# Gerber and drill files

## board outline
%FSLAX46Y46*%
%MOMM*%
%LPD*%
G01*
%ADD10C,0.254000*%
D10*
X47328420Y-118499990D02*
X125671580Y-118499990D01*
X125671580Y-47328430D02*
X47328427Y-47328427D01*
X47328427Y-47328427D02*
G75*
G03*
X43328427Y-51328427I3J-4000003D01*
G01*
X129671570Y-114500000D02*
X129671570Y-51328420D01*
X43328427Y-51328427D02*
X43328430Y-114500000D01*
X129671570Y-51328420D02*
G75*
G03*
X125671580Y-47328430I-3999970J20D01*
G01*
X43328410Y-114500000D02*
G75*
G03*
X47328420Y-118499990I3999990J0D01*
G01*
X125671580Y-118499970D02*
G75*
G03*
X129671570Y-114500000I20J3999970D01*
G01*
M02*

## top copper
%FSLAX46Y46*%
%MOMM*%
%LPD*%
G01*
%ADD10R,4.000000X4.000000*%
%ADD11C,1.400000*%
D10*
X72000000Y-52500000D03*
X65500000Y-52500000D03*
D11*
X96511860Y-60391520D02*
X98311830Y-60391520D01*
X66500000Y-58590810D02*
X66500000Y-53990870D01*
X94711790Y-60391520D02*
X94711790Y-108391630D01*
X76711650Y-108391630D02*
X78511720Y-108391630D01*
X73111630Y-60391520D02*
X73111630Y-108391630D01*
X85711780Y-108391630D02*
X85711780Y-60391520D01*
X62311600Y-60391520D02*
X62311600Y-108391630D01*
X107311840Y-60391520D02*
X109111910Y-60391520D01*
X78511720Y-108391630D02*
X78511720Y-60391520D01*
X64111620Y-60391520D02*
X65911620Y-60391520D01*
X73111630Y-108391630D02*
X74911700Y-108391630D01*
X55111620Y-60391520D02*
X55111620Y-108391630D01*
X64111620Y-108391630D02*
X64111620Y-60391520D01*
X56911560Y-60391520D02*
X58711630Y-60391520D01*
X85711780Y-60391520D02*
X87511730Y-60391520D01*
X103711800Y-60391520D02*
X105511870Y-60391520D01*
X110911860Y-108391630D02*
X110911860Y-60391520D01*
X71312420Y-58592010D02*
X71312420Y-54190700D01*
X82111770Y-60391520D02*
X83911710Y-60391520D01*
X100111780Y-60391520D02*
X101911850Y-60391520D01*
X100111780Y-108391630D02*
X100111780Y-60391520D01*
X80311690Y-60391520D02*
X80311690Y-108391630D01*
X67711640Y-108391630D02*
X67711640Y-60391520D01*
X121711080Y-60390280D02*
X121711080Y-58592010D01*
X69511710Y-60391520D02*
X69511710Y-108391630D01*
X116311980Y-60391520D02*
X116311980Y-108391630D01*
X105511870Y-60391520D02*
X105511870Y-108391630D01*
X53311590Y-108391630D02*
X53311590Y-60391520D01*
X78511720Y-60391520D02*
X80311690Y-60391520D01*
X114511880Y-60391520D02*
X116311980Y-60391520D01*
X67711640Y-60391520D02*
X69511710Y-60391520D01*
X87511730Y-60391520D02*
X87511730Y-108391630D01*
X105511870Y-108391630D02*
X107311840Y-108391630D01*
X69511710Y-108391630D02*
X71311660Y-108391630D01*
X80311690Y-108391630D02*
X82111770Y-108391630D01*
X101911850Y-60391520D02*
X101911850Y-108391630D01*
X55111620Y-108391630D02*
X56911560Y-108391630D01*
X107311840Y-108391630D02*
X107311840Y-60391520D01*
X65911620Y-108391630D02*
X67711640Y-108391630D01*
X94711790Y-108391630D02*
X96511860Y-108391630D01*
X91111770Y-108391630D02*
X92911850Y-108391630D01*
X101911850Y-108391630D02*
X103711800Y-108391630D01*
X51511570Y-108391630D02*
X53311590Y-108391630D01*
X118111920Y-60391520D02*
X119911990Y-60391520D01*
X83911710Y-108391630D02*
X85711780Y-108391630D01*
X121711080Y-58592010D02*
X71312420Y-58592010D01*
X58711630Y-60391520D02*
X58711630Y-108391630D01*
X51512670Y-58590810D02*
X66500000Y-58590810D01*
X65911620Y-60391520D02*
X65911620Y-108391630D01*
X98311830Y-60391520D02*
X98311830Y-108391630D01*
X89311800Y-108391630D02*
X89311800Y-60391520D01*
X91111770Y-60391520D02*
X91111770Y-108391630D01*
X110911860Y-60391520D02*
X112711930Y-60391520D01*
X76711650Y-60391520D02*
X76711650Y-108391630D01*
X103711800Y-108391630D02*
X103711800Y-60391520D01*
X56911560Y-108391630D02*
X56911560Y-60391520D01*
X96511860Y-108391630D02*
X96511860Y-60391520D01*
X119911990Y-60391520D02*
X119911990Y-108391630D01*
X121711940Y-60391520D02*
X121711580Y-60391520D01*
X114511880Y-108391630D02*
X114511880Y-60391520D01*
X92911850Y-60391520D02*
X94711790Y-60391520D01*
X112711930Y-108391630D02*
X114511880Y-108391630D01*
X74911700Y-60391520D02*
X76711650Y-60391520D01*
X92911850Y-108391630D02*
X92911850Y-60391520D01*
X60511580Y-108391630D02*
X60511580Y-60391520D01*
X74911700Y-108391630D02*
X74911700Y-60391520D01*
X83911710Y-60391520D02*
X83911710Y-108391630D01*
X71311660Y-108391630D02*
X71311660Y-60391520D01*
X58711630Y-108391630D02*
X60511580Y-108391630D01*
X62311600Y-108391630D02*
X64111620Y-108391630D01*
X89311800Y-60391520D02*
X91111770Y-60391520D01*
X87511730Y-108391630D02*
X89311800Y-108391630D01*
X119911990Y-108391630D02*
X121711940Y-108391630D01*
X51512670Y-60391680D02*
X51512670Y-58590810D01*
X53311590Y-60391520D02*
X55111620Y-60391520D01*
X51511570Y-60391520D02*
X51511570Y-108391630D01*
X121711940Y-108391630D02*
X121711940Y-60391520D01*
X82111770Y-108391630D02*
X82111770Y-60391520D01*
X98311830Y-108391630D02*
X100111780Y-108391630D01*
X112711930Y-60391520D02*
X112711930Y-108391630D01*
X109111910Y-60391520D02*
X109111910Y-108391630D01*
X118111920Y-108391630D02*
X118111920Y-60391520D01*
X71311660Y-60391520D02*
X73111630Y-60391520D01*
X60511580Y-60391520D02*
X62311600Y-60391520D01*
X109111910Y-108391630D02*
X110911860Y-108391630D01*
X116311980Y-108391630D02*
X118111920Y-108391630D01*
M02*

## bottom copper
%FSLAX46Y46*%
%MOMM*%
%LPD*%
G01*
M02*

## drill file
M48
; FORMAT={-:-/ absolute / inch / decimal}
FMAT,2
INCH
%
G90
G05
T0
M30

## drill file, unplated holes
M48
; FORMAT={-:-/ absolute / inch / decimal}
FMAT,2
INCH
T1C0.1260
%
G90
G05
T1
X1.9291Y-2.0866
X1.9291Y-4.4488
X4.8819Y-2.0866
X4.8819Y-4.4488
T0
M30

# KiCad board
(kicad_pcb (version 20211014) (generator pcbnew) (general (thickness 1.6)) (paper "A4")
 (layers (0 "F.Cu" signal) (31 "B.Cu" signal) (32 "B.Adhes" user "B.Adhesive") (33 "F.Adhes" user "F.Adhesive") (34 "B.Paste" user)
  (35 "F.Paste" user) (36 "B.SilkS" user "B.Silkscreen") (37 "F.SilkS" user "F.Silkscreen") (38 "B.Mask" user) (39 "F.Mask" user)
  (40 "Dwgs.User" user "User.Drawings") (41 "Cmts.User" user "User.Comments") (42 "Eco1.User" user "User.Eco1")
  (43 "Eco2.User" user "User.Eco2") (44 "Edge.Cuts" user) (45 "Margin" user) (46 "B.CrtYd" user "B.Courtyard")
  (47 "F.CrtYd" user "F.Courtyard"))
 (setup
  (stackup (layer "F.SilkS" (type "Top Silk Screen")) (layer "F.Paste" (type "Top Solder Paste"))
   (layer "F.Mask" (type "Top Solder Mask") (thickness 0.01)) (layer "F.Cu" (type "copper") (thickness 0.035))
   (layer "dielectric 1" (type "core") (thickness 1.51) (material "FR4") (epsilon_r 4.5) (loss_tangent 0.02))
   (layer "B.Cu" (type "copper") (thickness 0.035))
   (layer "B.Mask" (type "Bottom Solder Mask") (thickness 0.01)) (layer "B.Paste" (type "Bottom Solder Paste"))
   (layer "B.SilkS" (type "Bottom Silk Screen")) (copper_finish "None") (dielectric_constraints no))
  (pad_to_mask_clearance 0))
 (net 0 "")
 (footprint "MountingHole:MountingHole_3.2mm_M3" (layer "F.Cu") (at 124 53)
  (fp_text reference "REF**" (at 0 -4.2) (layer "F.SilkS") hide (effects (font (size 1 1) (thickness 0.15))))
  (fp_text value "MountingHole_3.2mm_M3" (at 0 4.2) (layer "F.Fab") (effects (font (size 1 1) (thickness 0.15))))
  (pad "" np_thru_hole circle (at 0 0) (size 3.2 3.2) (drill 3.2) (layers *.Cu *.Mask)))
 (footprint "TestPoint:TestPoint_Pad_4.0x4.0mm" (layer "F.Cu") (at 72 52.5)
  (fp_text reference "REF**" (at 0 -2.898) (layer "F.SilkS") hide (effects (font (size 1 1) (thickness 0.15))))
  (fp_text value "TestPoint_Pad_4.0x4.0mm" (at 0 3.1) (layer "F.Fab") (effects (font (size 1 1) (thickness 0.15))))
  (pad "1" smd rect (at 0 0) (size 4 4) (layers "F.Cu" "F.Mask")))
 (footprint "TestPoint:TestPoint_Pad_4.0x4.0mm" (layer "F.Cu") (at 65.5 52.5)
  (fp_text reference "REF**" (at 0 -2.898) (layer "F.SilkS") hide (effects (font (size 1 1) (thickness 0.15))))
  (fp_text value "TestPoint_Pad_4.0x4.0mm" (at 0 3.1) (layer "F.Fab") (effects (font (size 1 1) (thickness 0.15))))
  (pad "1" smd rect (at 0 0) (size 4 4) (layers "F.Cu" "F.Mask")))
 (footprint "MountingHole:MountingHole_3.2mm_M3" (layer "F.Cu") (at 49 113)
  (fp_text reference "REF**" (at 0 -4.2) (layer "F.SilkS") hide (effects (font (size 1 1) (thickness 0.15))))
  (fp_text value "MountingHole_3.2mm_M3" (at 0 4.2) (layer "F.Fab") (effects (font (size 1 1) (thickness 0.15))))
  (pad "" np_thru_hole circle (at 0 0) (size 3.2 3.2) (drill 3.2) (layers *.Cu *.Mask)))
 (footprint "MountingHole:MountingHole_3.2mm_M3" (layer "F.Cu") (at 124 113)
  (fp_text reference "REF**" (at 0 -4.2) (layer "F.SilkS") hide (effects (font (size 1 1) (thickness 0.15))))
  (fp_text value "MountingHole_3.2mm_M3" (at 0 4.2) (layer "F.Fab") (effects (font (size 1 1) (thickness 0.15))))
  (pad "" np_thru_hole circle (at 0 0) (size 3.2 3.2) (drill 3.2) (layers *.Cu *.Mask)))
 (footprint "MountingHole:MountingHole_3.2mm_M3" (layer "F.Cu") (at 49 53)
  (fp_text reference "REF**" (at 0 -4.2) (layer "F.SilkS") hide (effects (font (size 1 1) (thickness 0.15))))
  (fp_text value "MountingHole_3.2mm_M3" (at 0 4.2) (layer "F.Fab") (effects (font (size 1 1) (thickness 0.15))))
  (pad "" np_thru_hole circle (at 0 0) (size 3.2 3.2) (drill 3.2) (layers *.Cu *.Mask)))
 (gr_line (start 47.32842 118.49999) (end 125.67158 118.49999) (layer "Edge.Cuts") (width 0.254))
 (gr_line (start 125.67158 47.32843) (end 47.328427 47.328427) (layer "Edge.Cuts") (width 0.254))
 (gr_arc (start 43.328427 51.328427) (mid 44.5 48.5) (end 47.328427 47.328427) (layer "Edge.Cuts") (width 0.254))
 (gr_line (start 129.67157 114.5) (end 129.67157 51.32842) (layer "Edge.Cuts") (width 0.254))
 (gr_line (start 43.328427 51.328427) (end 43.32843 114.5) (layer "Edge.Cuts") (width 0.254))
 (gr_arc (start 125.67158 47.32843) (mid 128.5 48.5) (end 129.67157 51.32842) (layer "Edge.Cuts") (width 0.254))
 (gr_arc (start 47.32842 118.49999) (mid 44.5 117.32842) (end 43.32843 114.5) (layer "Edge.Cuts") (width 0.254))
 (gr_arc (start 129.67157 114.5) (mid 128.5 117.32842) (end 125.67158 118.49999) (layer "Edge.Cuts") (width 0.254))
 (segment (start 96.51186 60.39152) (end 98.31183 60.39152) (width 1.4) (layer "F.Cu") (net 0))
 (segment (start 66.5 58.59081) (end 66.5 53.99087) (width 1.4) (layer "F.Cu") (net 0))
 (segment (start 94.71179 60.39152) (end 94.71179 108.39163) (width 1.4) (layer "F.Cu") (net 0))
 (segment (start 76.71165 108.39163) (end 78.51172 108.39163) (width 1.4) (layer "F.Cu") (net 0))
 (segment (start 73.11163 60.39152) (end 73.11163 108.39163) (width 1.4) (layer "F.Cu") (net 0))
 (segment (start 85.71178 108.39163) (end 85.71178 60.39152) (width 1.4) (layer "F.Cu") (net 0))
 (segment (start 62.3116 60.39152) (end 62.3116 108.39163) (width 1.4) (layer "F.Cu") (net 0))
 (segment (start 107.31184 60.39152) (end 109.11191 60.39152) (width 1.4) (layer "F.Cu") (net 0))
 (segment (start 78.51172 108.39163) (end 78.51172 60.39152) (width 1.4) (layer "F.Cu") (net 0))
 (segment (start 64.11162 60.39152) (end 65.91162 60.39152) (width 1.4) (layer "F.Cu") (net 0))
 (segment (start 73.11163 108.39163) (end 74.9117 108.39163) (width 1.4) (layer "F.Cu") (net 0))
 (segment (start 55.11162 60.39152) (end 55.11162 108.39163) (width 1.4) (layer "F.Cu") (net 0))
 (segment (start 64.11162 108.39163) (end 64.11162 60.39152) (width 1.4) (layer "F.Cu") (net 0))
 (segment (start 56.91156 60.39152) (end 58.71163 60.39152) (width 1.4) (layer "F.Cu") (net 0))
 (segment (start 85.71178 60.39152) (end 87.51173 60.39152) (width 1.4) (layer "F.Cu") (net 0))
 (segment (start 103.7118 60.39152) (end 105.51187 60.39152) (width 1.4) (layer "F.Cu") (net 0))
 (segment (start 110.91186 108.39163) (end 110.91186 60.39152) (width 1.4) (layer "F.Cu") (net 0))
 (segment (start 71.31242 58.59201) (end 71.31242 54.1907) (width 1.4) (layer "F.Cu") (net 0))
 (segment (start 82.11177 60.39152) (end 83.91171 60.39152) (width 1.4) (layer "F.Cu") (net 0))
 (segment (start 100.11178 60.39152) (end 101.91185 60.39152) (width 1.4) (layer "F.Cu") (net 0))
 (segment (start 100.11178 108.39163) (end 100.11178 60.39152) (width 1.4) (layer "F.Cu") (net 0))
 (segment (start 80.31169 60.39152) (end 80.31169 108.39163) (width 1.4) (layer "F.Cu") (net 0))
 (segment (start 67.71164 108.39163) (end 67.71164 60.39152) (width 1.4) (layer "F.Cu") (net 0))
 (segment (start 121.71108 60.39028) (end 121.71108 58.59201) (width 1.4) (layer "F.Cu") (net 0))
 (segment (start 69.51171 60.39152) (end 69.51171 108.39163) (width 1.4) (layer "F.Cu") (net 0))
 (segment (start 116.31198 60.39152) (end 116.31198 108.39163) (width 1.4) (layer "F.Cu") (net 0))
 (segment (start 105.51187 60.39152) (end 105.51187 108.39163) (width 1.4) (layer "F.Cu") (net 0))
 (segment (start 53.31159 108.39163) (end 53.31159 60.39152) (width 1.4) (layer "F.Cu") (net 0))
 (segment (start 78.51172 60.39152) (end 80.31169 60.39152) (width 1.4) (layer "F.Cu") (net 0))
 (segment (start 114.51188 60.39152) (end 116.31198 60.39152) (width 1.4) (layer "F.Cu") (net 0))
 (segment (start 67.71164 60.39152) (end 69.51171 60.39152) (width 1.4) (layer "F.Cu") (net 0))
 (segment (start 87.51173 60.39152) (end 87.51173 108.39163) (width 1.4) (layer "F.Cu") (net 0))
 (segment (start 105.51187 108.39163) (end 107.31184 108.39163) (width 1.4) (layer "F.Cu") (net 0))
 (segment (start 69.51171 108.39163) (end 71.31166 108.39163) (width 1.4) (layer "F.Cu") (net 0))
 (segment (start 80.31169 108.39163) (end 82.11177 108.39163) (width 1.4) (layer "F.Cu") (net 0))
 (segment (start 101.91185 60.39152) (end 101.91185 108.39163) (width 1.4) (layer "F.Cu") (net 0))
 (segment (start 55.11162 108.39163) (end 56.91156 108.39163) (width 1.4) (layer "F.Cu") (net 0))
 (segment (start 107.31184 108.39163) (end 107.31184 60.39152) (width 1.4) (layer "F.Cu") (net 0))
 (segment (start 65.91162 108.39163) (end 67.71164 108.39163) (width 1.4) (layer "F.Cu") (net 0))
 (segment (start 94.71179 108.39163) (end 96.51186 108.39163) (width 1.4) (layer "F.Cu") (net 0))
 (segment (start 91.11177 108.39163) (end 92.91185 108.39163) (width 1.4) (layer "F.Cu") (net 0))
 (segment (start 101.91185 108.39163) (end 103.7118 108.39163) (width 1.4) (layer "F.Cu") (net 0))
 (segment (start 51.51157 108.39163) (end 53.31159 108.39163) (width 1.4) (layer "F.Cu") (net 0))
 (segment (start 118.11192 60.39152) (end 119.91199 60.39152) (width 1.4) (layer "F.Cu") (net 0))
 (segment (start 83.91171 108.39163) (end 85.71178 108.39163) (width 1.4) (layer "F.Cu") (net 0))
 (segment (start 121.71108 58.59201) (end 71.31242 58.59201) (width 1.4) (layer "F.Cu") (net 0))
 (segment (start 58.71163 60.39152) (end 58.71163 108.39163) (width 1.4) (layer "F.Cu") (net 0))
 (segment (start 51.51267 58.59081) (end 66.5 58.59081) (width 1.4) (layer "F.Cu") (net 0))
 (segment (start 65.91162 60.39152) (end 65.91162 108.39163) (width 1.4) (layer "F.Cu") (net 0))
 (segment (start 98.31183 60.39152) (end 98.31183 108.39163) (width 1.4) (layer "F.Cu") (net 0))
 (segment (start 89.3118 108.39163) (end 89.3118 60.39152) (width 1.4) (layer "F.Cu") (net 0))
 (segment (start 91.11177 60.39152) (end 91.11177 108.39163) (width 1.4) (layer "F.Cu") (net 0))
 (segment (start 110.91186 60.39152) (end 112.71193 60.39152) (width 1.4) (layer "F.Cu") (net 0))
 (segment (start 76.71165 60.39152) (end 76.71165 108.39163) (width 1.4) (layer "F.Cu") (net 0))
 (segment (start 103.7118 108.39163) (end 103.7118 60.39152) (width 1.4) (layer "F.Cu") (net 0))
 (segment (start 56.91156 108.39163) (end 56.91156 60.39152) (width 1.4) (layer "F.Cu") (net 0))
 (segment (start 96.51186 108.39163) (end 96.51186 60.39152) (width 1.4) (layer "F.Cu") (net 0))
 (segment (start 119.91199 60.39152) (end 119.91199 108.39163) (width 1.4) (layer "F.Cu") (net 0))
 (segment (start 121.71194 60.39152) (end 121.71158 60.39152) (width 1.4) (layer "F.Cu") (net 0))
 (segment (start 114.51188 108.39163) (end 114.51188 60.39152) (width 1.4) (layer "F.Cu") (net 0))
 (segment (start 92.91185 60.39152) (end 94.71179 60.39152) (width 1.4) (layer "F.Cu") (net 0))
 (segment (start 112.71193 108.39163) (end 114.51188 108.39163) (width 1.4) (layer "F.Cu") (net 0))
 (segment (start 74.9117 60.39152) (end 76.71165 60.39152) (width 1.4) (layer "F.Cu") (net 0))
 (segment (start 92.91185 108.39163) (end 92.91185 60.39152) (width 1.4) (layer "F.Cu") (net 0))
 (segment (start 60.51158 108.39163) (end 60.51158 60.39152) (width 1.4) (layer "F.Cu") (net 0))
 (segment (start 74.9117 108.39163) (end 74.9117 60.39152) (width 1.4) (layer "F.Cu") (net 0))
 (segment (start 83.91171 60.39152) (end 83.91171 108.39163) (width 1.4) (layer "F.Cu") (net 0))
 (segment (start 71.31166 108.39163) (end 71.31166 60.39152) (width 1.4) (layer "F.Cu") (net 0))
 (segment (start 58.71163 108.39163) (end 60.51158 108.39163) (width 1.4) (layer "F.Cu") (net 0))
 (segment (start 62.3116 108.39163) (end 64.11162 108.39163) (width 1.4) (layer "F.Cu") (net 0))
 (segment (start 89.3118 60.39152) (end 91.11177 60.39152) (width 1.4) (layer "F.Cu") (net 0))
 (segment (start 87.51173 108.39163) (end 89.3118 108.39163) (width 1.4) (layer "F.Cu") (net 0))
 (segment (start 119.91199 108.39163) (end 121.71194 108.39163) (width 1.4) (layer "F.Cu") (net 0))
 (segment (start 51.51267 60.39168) (end 51.51267 58.59081) (width 1.4) (layer "F.Cu") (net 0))
 (segment (start 53.31159 60.39152) (end 55.11162 60.39152) (width 1.4) (layer "F.Cu") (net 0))
 (segment (start 51.51157 60.39152) (end 51.51157 108.39163) (width 1.4) (layer "F.Cu") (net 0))
 (segment (start 121.71194 108.39163) (end 121.71194 60.39152) (width 1.4) (layer "F.Cu") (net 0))
 (segment (start 82.11177 108.39163) (end 82.11177 60.39152) (width 1.4) (layer "F.Cu") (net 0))
 (segment (start 98.31183 108.39163) (end 100.11178 108.39163) (width 1.4) (layer "F.Cu") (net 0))
 (segment (start 112.71193 60.39152) (end 112.71193 108.39163) (width 1.4) (layer "F.Cu") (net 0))
 (segment (start 109.11191 60.39152) (end 109.11191 108.39163) (width 1.4) (layer "F.Cu") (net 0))
 (segment (start 118.11192 108.39163) (end 118.11192 60.39152) (width 1.4) (layer "F.Cu") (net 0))
 (segment (start 71.31166 60.39152) (end 73.11163 60.39152) (width 1.4) (layer "F.Cu") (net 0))
 (segment (start 60.51158 60.39152) (end 62.3116 60.39152) (width 1.4) (layer "F.Cu") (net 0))
 (segment (start 109.11191 108.39163) (end 110.91186 108.39163) (width 1.4) (layer "F.Cu") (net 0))
 (segment (start 116.31198 108.39163) (end 118.11192 108.39163) (width 1.4) (layer "F.Cu") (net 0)))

